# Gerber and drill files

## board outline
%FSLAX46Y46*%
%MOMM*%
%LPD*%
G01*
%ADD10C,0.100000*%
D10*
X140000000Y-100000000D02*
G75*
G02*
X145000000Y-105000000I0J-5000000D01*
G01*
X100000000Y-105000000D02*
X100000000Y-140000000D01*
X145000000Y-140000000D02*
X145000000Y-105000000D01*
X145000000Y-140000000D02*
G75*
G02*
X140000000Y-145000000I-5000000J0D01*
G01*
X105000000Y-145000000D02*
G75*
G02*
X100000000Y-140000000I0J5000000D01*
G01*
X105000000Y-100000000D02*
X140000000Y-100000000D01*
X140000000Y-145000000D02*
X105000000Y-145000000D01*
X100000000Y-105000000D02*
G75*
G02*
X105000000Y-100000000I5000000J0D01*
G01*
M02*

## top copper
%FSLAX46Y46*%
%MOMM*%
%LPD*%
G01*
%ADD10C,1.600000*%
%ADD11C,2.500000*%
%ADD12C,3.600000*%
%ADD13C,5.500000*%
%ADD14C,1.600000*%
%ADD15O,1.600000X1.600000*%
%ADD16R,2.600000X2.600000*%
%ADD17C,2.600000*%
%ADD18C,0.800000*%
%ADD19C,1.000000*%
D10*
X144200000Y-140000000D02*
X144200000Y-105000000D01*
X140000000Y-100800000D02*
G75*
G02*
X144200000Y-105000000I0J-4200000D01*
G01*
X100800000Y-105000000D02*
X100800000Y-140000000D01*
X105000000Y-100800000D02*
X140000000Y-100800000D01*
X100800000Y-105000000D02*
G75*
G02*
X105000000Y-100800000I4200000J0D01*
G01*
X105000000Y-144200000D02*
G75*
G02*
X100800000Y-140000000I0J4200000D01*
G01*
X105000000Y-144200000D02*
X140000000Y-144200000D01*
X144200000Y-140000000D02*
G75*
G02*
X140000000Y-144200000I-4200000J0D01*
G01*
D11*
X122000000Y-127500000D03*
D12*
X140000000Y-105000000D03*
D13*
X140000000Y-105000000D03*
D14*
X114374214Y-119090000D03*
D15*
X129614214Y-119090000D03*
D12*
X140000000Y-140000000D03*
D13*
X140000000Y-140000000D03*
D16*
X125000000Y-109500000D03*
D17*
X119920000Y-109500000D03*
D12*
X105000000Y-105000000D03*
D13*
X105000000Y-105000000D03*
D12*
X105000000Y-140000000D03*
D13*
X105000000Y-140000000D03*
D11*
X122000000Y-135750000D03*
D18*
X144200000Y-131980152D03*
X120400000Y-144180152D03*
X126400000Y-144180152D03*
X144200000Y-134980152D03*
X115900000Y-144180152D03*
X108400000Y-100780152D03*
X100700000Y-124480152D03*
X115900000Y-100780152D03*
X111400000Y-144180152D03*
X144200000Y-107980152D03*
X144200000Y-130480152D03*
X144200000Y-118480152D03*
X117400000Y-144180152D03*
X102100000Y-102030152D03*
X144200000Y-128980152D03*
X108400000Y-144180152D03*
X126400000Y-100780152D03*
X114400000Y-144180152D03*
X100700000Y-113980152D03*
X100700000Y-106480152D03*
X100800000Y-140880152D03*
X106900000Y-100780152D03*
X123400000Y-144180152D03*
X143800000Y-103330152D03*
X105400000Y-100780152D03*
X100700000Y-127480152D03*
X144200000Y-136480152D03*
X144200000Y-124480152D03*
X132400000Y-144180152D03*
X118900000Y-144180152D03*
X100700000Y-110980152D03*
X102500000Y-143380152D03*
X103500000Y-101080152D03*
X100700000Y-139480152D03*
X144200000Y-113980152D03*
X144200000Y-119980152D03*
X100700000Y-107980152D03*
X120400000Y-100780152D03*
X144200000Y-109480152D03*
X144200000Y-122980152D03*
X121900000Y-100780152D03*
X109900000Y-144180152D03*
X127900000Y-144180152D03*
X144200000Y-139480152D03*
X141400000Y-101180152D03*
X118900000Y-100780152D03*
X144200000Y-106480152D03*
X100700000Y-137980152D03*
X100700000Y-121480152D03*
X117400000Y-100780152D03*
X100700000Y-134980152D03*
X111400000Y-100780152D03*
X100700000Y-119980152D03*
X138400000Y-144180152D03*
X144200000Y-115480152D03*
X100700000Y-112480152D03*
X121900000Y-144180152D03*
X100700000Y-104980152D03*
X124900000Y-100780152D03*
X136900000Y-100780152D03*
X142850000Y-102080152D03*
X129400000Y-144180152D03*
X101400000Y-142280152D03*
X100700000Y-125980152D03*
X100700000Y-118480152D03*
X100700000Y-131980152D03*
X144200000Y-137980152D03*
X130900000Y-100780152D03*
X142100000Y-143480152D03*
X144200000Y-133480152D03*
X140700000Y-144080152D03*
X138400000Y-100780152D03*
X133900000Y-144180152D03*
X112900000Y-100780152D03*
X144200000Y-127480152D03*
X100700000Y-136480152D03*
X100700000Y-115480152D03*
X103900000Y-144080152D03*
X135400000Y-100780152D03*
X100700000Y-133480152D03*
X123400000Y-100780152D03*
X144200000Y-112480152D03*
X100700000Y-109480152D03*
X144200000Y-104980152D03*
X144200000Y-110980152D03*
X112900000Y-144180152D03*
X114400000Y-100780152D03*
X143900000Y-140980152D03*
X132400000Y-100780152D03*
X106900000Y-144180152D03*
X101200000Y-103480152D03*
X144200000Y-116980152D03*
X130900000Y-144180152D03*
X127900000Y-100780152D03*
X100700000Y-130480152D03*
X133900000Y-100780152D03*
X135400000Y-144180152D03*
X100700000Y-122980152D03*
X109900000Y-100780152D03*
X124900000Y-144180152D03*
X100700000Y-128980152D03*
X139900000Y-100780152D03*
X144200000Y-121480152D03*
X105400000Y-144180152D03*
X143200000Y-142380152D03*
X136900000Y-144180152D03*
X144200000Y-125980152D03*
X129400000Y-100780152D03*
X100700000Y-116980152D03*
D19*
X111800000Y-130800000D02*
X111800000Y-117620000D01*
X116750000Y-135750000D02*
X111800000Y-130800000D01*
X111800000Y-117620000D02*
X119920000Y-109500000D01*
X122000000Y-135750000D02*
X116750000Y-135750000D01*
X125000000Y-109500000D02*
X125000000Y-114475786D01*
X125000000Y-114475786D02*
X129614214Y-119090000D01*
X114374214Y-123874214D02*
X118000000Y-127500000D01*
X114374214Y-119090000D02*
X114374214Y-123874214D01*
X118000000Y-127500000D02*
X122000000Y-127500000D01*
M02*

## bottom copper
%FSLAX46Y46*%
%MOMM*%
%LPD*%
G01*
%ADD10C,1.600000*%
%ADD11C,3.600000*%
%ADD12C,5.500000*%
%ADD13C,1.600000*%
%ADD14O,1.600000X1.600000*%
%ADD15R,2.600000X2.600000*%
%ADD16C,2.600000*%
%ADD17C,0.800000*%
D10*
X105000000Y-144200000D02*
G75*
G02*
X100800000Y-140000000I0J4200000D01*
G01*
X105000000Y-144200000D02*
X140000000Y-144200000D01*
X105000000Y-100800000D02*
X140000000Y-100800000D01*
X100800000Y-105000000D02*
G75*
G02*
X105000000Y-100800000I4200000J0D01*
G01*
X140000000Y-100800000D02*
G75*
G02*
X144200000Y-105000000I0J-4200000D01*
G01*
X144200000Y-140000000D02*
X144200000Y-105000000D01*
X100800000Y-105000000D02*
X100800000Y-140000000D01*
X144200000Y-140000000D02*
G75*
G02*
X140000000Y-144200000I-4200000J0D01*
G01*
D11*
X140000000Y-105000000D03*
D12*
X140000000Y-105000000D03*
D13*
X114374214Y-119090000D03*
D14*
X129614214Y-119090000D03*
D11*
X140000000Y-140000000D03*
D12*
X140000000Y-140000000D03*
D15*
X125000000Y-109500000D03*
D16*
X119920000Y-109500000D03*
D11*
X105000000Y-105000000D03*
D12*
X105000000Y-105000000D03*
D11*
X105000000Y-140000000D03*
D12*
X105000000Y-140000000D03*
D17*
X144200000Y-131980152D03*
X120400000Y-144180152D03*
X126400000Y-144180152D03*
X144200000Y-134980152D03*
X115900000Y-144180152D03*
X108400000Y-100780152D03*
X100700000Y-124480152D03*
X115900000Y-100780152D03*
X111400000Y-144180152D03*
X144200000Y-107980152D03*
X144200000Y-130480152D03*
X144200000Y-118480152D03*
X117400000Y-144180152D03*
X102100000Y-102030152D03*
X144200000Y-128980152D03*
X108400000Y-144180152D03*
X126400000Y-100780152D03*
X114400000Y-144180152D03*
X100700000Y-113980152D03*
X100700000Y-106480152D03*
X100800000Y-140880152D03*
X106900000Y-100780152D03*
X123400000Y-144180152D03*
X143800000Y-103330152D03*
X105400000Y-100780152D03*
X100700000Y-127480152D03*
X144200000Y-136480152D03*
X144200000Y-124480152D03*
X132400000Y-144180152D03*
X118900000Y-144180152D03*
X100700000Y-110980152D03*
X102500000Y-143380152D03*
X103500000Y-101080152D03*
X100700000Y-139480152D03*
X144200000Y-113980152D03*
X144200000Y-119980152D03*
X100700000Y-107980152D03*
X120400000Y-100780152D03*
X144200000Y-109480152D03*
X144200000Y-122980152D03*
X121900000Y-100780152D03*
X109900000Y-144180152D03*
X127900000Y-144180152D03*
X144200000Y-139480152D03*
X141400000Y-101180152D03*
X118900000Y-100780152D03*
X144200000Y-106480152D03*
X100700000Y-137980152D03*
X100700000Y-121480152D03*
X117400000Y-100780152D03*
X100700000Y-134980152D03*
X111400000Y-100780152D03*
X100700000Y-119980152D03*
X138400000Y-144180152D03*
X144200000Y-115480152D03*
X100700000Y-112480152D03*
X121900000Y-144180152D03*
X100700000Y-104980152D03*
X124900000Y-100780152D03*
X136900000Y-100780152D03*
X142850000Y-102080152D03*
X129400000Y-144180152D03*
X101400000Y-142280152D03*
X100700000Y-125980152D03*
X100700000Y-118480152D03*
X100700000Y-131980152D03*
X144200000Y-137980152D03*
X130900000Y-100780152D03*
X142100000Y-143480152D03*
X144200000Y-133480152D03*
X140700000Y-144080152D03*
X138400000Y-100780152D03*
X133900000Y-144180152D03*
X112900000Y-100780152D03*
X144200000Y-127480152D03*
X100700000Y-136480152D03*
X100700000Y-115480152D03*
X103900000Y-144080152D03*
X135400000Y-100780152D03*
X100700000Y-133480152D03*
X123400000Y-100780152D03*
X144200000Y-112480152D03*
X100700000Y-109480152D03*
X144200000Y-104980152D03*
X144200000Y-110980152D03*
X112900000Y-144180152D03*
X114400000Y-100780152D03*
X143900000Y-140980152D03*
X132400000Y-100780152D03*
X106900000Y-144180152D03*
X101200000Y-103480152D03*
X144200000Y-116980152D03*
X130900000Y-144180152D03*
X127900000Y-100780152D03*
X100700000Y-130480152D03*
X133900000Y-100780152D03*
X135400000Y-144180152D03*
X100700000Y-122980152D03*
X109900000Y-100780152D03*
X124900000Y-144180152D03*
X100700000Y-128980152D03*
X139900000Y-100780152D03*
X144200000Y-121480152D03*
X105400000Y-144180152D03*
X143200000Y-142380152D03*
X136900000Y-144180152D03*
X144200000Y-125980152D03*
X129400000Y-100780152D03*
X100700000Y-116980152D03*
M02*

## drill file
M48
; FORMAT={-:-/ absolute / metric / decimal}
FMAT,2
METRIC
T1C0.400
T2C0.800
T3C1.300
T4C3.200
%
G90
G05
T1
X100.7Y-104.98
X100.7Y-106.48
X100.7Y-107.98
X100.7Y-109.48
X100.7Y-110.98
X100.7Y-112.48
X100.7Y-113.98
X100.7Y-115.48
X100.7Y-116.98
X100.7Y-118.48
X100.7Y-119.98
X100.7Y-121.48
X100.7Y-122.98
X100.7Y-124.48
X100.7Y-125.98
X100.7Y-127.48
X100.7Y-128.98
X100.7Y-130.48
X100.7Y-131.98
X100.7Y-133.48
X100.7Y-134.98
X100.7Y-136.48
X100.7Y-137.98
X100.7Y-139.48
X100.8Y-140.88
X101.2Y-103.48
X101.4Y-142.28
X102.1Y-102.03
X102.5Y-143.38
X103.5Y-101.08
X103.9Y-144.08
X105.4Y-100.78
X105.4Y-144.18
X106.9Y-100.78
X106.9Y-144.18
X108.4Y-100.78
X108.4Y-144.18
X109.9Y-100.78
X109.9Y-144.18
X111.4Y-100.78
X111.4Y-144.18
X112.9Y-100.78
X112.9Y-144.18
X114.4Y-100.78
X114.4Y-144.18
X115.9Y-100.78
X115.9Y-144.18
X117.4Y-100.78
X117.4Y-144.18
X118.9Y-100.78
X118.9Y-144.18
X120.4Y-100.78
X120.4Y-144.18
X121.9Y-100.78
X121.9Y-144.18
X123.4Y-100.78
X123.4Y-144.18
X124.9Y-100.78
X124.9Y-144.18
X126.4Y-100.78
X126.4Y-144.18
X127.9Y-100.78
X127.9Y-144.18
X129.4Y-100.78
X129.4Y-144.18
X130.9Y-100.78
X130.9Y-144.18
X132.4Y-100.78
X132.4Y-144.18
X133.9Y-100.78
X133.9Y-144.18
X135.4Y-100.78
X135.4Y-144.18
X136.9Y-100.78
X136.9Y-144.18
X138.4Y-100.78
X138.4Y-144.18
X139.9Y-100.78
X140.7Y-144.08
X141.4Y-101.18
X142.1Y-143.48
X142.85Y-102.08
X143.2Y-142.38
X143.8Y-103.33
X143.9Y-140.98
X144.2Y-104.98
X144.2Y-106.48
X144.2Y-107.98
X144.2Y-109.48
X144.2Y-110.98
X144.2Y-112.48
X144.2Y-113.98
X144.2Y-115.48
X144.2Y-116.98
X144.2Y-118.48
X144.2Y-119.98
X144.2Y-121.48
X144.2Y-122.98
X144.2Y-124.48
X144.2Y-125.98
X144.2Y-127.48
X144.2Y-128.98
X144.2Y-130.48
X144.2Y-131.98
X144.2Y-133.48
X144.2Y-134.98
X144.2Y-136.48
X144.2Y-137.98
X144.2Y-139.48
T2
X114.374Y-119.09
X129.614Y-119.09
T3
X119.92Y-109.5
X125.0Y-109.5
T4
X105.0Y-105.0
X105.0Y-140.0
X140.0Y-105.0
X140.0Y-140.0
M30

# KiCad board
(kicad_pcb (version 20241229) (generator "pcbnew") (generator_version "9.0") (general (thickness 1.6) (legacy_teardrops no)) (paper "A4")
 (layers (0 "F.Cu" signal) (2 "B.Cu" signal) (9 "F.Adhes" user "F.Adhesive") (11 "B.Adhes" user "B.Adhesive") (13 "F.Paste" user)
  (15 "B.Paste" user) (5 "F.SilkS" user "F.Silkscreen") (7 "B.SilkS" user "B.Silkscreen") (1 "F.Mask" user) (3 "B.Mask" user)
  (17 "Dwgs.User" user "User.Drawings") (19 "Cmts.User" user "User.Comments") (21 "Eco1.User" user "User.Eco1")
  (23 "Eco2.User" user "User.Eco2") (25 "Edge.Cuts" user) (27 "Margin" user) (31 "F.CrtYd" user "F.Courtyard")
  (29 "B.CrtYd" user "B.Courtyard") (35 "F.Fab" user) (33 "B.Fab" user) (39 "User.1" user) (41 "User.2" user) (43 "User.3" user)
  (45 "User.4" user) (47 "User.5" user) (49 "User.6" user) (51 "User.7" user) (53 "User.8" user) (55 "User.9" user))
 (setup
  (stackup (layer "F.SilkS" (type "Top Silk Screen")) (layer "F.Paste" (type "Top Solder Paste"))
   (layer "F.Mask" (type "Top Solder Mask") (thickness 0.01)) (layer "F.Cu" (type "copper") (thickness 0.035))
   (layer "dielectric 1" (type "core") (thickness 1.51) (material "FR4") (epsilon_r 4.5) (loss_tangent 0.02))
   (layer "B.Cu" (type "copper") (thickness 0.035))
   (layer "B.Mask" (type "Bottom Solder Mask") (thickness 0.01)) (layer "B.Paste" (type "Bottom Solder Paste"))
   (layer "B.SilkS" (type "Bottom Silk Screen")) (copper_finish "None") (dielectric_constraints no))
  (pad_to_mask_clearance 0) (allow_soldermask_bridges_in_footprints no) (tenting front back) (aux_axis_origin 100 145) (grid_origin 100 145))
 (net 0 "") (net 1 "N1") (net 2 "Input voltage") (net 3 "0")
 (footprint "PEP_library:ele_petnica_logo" (layer "F.Cu") (at 136 126.6)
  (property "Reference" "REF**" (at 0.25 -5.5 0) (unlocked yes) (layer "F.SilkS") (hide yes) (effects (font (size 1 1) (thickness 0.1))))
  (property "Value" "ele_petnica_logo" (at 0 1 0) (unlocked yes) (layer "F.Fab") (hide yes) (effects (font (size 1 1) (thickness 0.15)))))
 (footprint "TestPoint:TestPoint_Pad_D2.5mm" (layer "F.Cu") (at 122 127.5)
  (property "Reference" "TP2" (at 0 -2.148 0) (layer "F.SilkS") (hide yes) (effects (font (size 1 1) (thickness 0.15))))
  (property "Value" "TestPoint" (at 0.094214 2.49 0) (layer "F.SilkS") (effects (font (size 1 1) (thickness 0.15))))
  (pad "1" smd circle (at 0 0) (size 2.5 2.5) (layers "F.Cu" "F.Mask") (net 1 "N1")))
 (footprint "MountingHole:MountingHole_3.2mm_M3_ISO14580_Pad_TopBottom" (layer "F.Cu") (at 140 105)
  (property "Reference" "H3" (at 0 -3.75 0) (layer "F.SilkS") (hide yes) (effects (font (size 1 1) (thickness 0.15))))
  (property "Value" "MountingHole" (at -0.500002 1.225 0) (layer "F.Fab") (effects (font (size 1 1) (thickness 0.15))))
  (pad "1" thru_hole circle (at 0 0) (size 3.6 3.6) (drill 3.2) (layers "*.Cu" "*.Mask") (remove_unused_layers no))
  (pad "1" connect circle (at 0 0) (size 5.5 5.5) (layers "F.Cu" "F.Mask"))
  (pad "1" connect circle (at 0 0) (size 5.5 5.5) (layers "B.Cu" "B.Mask")))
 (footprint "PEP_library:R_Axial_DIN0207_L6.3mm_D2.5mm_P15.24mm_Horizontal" (layer "F.Cu") (at 114.374214 119.09)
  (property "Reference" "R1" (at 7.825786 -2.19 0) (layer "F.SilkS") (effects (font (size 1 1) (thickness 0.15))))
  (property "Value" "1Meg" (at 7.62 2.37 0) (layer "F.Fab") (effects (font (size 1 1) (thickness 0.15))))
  (pad "1" thru_hole circle (at 0 0) (size 1.6 1.6) (drill 0.8) (layers "*.Cu" "*.Mask") (remove_unused_layers no) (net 1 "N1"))
  (pad "2" thru_hole oval (at 15.24 0) (size 1.6 1.6) (drill 0.8) (layers "*.Cu" "*.Mask") (remove_unused_layers no) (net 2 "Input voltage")))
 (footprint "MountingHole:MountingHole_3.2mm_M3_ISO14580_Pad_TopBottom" (layer "F.Cu") (at 140 140)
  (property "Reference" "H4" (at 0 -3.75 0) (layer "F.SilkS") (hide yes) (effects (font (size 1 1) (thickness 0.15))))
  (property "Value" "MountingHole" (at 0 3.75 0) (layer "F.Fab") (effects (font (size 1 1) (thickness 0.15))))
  (pad "1" thru_hole circle (at 0 0) (size 3.6 3.6) (drill 3.2) (layers "*.Cu" "*.Mask") (remove_unused_layers no))
  (pad "1" connect circle (at 0 0) (size 5.5 5.5) (layers "F.Cu" "F.Mask"))
  (pad "1" connect circle (at 0 0) (size 5.5 5.5) (layers "B.Cu" "B.Mask")))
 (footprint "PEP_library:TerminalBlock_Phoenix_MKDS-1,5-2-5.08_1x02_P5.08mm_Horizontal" (layer "F.Cu") (at 125 109.5 180)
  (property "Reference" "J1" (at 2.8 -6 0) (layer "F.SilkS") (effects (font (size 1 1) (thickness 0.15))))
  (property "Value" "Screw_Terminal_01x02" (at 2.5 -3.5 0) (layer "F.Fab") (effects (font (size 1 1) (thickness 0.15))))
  (pad "1" thru_hole rect (at 0 0 180) (size 2.6 2.6) (drill 1.3) (layers "*.Cu" "*.Mask") (remove_unused_layers no) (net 2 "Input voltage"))
  (pad "2" thru_hole circle (at 5.08 0 180) (size 2.6 2.6) (drill 1.3) (layers "*.Cu" "*.Mask") (remove_unused_layers no) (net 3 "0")))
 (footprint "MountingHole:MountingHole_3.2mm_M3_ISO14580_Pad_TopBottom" (layer "F.Cu") (at 105 105)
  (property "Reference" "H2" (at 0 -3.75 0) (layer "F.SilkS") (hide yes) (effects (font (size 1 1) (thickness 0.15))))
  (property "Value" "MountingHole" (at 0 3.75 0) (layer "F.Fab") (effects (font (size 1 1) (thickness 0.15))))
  (pad "1" thru_hole circle (at 0 0) (size 3.6 3.6) (drill 3.2) (layers "*.Cu" "*.Mask") (remove_unused_layers no))
  (pad "1" connect circle (at 0 0) (size 5.5 5.5) (layers "F.Cu" "F.Mask"))
  (pad "1" connect circle (at 0 0) (size 5.5 5.5) (layers "B.Cu" "B.Mask")))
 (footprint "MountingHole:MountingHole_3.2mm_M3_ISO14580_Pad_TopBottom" (layer "F.Cu") (at 105 140 -90)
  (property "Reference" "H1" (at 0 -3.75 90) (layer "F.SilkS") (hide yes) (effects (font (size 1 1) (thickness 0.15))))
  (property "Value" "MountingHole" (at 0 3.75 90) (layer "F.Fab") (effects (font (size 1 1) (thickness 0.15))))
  (pad "1" thru_hole circle (at 0 0 270) (size 3.6 3.6) (drill 3.2) (layers "*.Cu" "*.Mask") (remove_unused_layers no))
  (pad "1" connect circle (at 0 0 270) (size 5.5 5.5) (layers "F.Cu" "F.Mask"))
  (pad "1" connect circle (at 0 0 270) (size 5.5 5.5) (layers "B.Cu" "B.Mask")))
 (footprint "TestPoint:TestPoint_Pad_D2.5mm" (layer "F.Cu") (at 122 135.75)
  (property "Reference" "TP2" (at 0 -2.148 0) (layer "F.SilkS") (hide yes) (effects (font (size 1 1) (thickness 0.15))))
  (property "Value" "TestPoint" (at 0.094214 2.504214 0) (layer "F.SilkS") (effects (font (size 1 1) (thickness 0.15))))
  (pad "2" smd circle (at 0 0) (size 2.5 2.5) (layers "F.Cu" "F.Mask") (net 3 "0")))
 (gr_line (start 144.2 140) (end 144.2 105) (stroke (width 1.6) (type default)) (locked yes) (layer "F.Cu"))
 (gr_arc (start 140 100.8) (mid 142.969848 102.030152) (end 144.2 105) (stroke (width 1.6) (type default)) (locked yes) (layer "F.Cu"))
 (gr_line (start 100.8 105) (end 100.8 140) (stroke (width 1.6) (type default)) (locked yes) (layer "F.Cu"))
 (gr_line (start 105 100.8) (end 140 100.8) (stroke (width 1.6) (type default)) (locked yes) (layer "F.Cu"))
 (gr_arc (start 100.8 105) (mid 102.030152 102.030152) (end 105 100.8) (stroke (width 1.6) (type default)) (locked yes) (layer "F.Cu"))
 (gr_arc (start 105 144.2) (mid 102.030152 142.969848) (end 100.8 140) (stroke (width 1.6) (type default)) (locked yes) (layer "F.Cu"))
 (gr_line (start 105 144.2) (end 140 144.2) (stroke (width 1.6) (type default)) (locked yes) (layer "F.Cu"))
 (gr_arc (start 144.2 140) (mid 142.969848 142.969848) (end 140 144.2) (stroke (width 1.6) (type default)) (locked yes) (layer "F.Cu"))
 (gr_arc (start 105 144.2) (mid 102.030154 142.969848) (end 100.8 140) (stroke (width 1.6) (type default)) (locked yes) (layer "B.Cu"))
 (gr_line (start 105 144.2) (end 140 144.2) (stroke (width 1.6) (type default)) (locked yes) (layer "B.Cu"))
 (gr_line (start 105 100.8) (end 140 100.8) (stroke (width 1.6) (type default)) (locked yes) (layer "B.Cu"))
 (gr_arc (start 100.8 105) (mid 102.030152 102.030152) (end 105 100.8) (stroke (width 1.6) (type default)) (locked yes) (layer "B.Cu"))
 (gr_arc (start 140 100.8) (mid 142.96985 102.030151) (end 144.2 105) (stroke (width 1.6) (type default)) (locked yes) (layer "B.Cu"))
 (gr_line (start 144.2 140) (end 144.2 105) (stroke (width 1.6) (type default)) (locked yes) (layer "B.Cu"))
 (gr_line (start 100.8 105) (end 100.8 140) (stroke (width 1.6) (type default)) (locked yes) (layer "B.Cu"))
 (gr_arc (start 144.2 140) (mid 142.969849 142.969849) (end 140 144.2) (stroke (width 1.6) (type default)) (locked yes) (layer "B.Cu"))
 (gr_arc (start 140 100) (mid 143.535534 101.464466) (end 145 105) (stroke (width 0.1) (type default)) (locked yes) (layer "Edge.Cuts"))
 (gr_line (start 100 105) (end 100 140) (stroke (width 0.1) (type default)) (locked yes) (layer "Edge.Cuts"))
 (gr_line (start 145 140) (end 145 105) (stroke (width 0.1) (type default)) (locked yes) (layer "Edge.Cuts"))
 (gr_arc (start 145 140) (mid 143.535534 143.535534) (end 140 145) (stroke (width 0.1) (type default)) (locked yes) (layer "Edge.Cuts"))
 (gr_arc (start 105 145) (mid 101.464466 143.535534) (end 100 140) (stroke (width 0.1) (type default)) (locked yes) (layer "Edge.Cuts"))
 (gr_line (start 105 100) (end 140 100) (stroke (width 0.1) (type default)) (locked yes) (layer "Edge.Cuts"))
 (gr_line (start 140 145) (end 105 145) (stroke (width 0.1) (type default)) (locked yes) (layer "Edge.Cuts"))
 (gr_arc (start 100 105) (mid 101.464466 101.464466) (end 105 100) (stroke (width 0.1) (type default)) (locked yes) (layer "Edge.Cuts"))
 (via (at 144.2 131.980152) (size 0.8) (drill 0.4) (layers "F.Cu" "B.Cu") (locked yes) (free yes) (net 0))
 (via (at 120.4 144.180152) (size 0.8) (drill 0.4) (layers "F.Cu" "B.Cu") (locked yes) (free yes) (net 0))
 (via (at 126.4 144.180152) (size 0.8) (drill 0.4) (layers "F.Cu" "B.Cu") (locked yes) (free yes) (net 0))
 (via (at 144.2 134.980152) (size 0.8) (drill 0.4) (layers "F.Cu" "B.Cu") (locked yes) (free yes) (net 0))
 (via (at 115.9 144.180152) (size 0.8) (drill 0.4) (layers "F.Cu" "B.Cu") (locked yes) (free yes) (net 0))
 (via (at 108.4 100.780152) (size 0.8) (drill 0.4) (layers "F.Cu" "B.Cu") (locked yes) (free yes) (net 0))
 (via (at 100.7 124.480152) (size 0.8) (drill 0.4) (layers "F.Cu" "B.Cu") (locked yes) (free yes) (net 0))
 (via (at 115.9 100.780152) (size 0.8) (drill 0.4) (layers "F.Cu" "B.Cu") (locked yes) (free yes) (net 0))
 (via (at 111.4 144.180152) (size 0.8) (drill 0.4) (layers "F.Cu" "B.Cu") (locked yes) (free yes) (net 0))
 (via (at 144.2 107.980152) (size 0.8) (drill 0.4) (layers "F.Cu" "B.Cu") (locked yes) (free yes) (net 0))
 (via (at 144.2 130.480152) (size 0.8) (drill 0.4) (layers "F.Cu" "B.Cu") (locked yes) (free yes) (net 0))
 (via (at 144.2 118.480152) (size 0.8) (drill 0.4) (layers "F.Cu" "B.Cu") (locked yes) (free yes) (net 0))
 (via (at 117.4 144.180152) (size 0.8) (drill 0.4) (layers "F.Cu" "B.Cu") (locked yes) (free yes) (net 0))
 (via (at 102.1 102.030152) (size 0.8) (drill 0.4) (layers "F.Cu" "B.Cu") (locked yes) (free yes) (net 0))
 (via (at 144.2 128.980152) (size 0.8) (drill 0.4) (layers "F.Cu" "B.Cu") (locked yes) (free yes) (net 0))
 (via (at 108.4 144.180152) (size 0.8) (drill 0.4) (layers "F.Cu" "B.Cu") (locked yes) (free yes) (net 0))
 (via (at 126.4 100.780152) (size 0.8) (drill 0.4) (layers "F.Cu" "B.Cu") (locked yes) (free yes) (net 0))
 (via (at 114.4 144.180152) (size 0.8) (drill 0.4) (layers "F.Cu" "B.Cu") (locked yes) (free yes) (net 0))
 (via (at 100.7 113.980152) (size 0.8) (drill 0.4) (layers "F.Cu" "B.Cu") (locked yes) (free yes) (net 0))
 (via (at 100.7 106.480152) (size 0.8) (drill 0.4) (layers "F.Cu" "B.Cu") (locked yes) (free yes) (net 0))
 (via (at 100.8 140.880152) (size 0.8) (drill 0.4) (layers "F.Cu" "B.Cu") (locked yes) (free yes) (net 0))
 (via (at 106.9 100.780152) (size 0.8) (drill 0.4) (layers "F.Cu" "B.Cu") (locked yes) (free yes) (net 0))
 (via (at 123.4 144.180152) (size 0.8) (drill 0.4) (layers "F.Cu" "B.Cu") (locked yes) (free yes) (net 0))
 (via (at 143.8 103.330152) (size 0.8) (drill 0.4) (layers "F.Cu" "B.Cu") (locked yes) (free yes) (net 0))
 (via (at 105.4 100.780152) (size 0.8) (drill 0.4) (layers "F.Cu" "B.Cu") (locked yes) (free yes) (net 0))
 (via (at 100.7 127.480152) (size 0.8) (drill 0.4) (layers "F.Cu" "B.Cu") (locked yes) (free yes) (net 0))
 (via (at 144.2 136.480152) (size 0.8) (drill 0.4) (layers "F.Cu" "B.Cu") (locked yes) (free yes) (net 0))
 (via (at 144.2 124.480152) (size 0.8) (drill 0.4) (layers "F.Cu" "B.Cu") (locked yes) (free yes) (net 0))
 (via (at 132.4 144.180152) (size 0.8) (drill 0.4) (layers "F.Cu" "B.Cu") (locked yes) (free yes) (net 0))
 (via (at 118.9 144.180152) (size 0.8) (drill 0.4) (layers "F.Cu" "B.Cu") (locked yes) (free yes) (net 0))
 (via (at 100.7 110.980152) (size 0.8) (drill 0.4) (layers "F.Cu" "B.Cu") (locked yes) (free yes) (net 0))
 (via (at 102.5 143.380152) (size 0.8) (drill 0.4) (layers "F.Cu" "B.Cu") (locked yes) (free yes) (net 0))
 (via (at 103.5 101.080152) (size 0.8) (drill 0.4) (layers "F.Cu" "B.Cu") (locked yes) (free yes) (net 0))
 (via (at 100.7 139.480152) (size 0.8) (drill 0.4) (layers "F.Cu" "B.Cu") (locked yes) (free yes) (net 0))
 (via (at 144.2 113.980152) (size 0.8) (drill 0.4) (layers "F.Cu" "B.Cu") (locked yes) (free yes) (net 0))
 (via (at 144.2 119.980152) (size 0.8) (drill 0.4) (layers "F.Cu" "B.Cu") (locked yes) (free yes) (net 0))
 (via (at 100.7 107.980152) (size 0.8) (drill 0.4) (layers "F.Cu" "B.Cu") (locked yes) (free yes) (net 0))
 (via (at 120.4 100.780152) (size 0.8) (drill 0.4) (layers "F.Cu" "B.Cu") (locked yes) (free yes) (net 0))
 (via (at 144.2 109.480152) (size 0.8) (drill 0.4) (layers "F.Cu" "B.Cu") (locked yes) (free yes) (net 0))
 (via (at 144.2 122.980152) (size 0.8) (drill 0.4) (layers "F.Cu" "B.Cu") (locked yes) (free yes) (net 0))
 (via (at 121.9 100.780152) (size 0.8) (drill 0.4) (layers "F.Cu" "B.Cu") (locked yes) (free yes) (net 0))
 (via (at 109.9 144.180152) (size 0.8) (drill 0.4) (layers "F.Cu" "B.Cu") (locked yes) (free yes) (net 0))
 (via (at 127.9 144.180152) (size 0.8) (drill 0.4) (layers "F.Cu" "B.Cu") (locked yes) (free yes) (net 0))
 (via (at 144.2 139.480152) (size 0.8) (drill 0.4) (layers "F.Cu" "B.Cu") (locked yes) (free yes) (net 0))
 (via (at 141.4 101.180152) (size 0.8) (drill 0.4) (layers "F.Cu" "B.Cu") (locked yes) (free yes) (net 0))
 (via (at 118.9 100.780152) (size 0.8) (drill 0.4) (layers "F.Cu" "B.Cu") (locked yes) (free yes) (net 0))
 (via (at 144.2 106.480152) (size 0.8) (drill 0.4) (layers "F.Cu" "B.Cu") (locked yes) (free yes) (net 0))
 (via (at 100.7 137.980152) (size 0.8) (drill 0.4) (layers "F.Cu" "B.Cu") (locked yes) (free yes) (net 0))
 (via (at 100.7 121.480152) (size 0.8) (drill 0.4) (layers "F.Cu" "B.Cu") (locked yes) (free yes) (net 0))
 (via (at 117.4 100.780152) (size 0.8) (drill 0.4) (layers "F.Cu" "B.Cu") (locked yes) (free yes) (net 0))
 (via (at 100.7 134.980152) (size 0.8) (drill 0.4) (layers "F.Cu" "B.Cu") (locked yes) (free yes) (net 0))
 (via (at 111.4 100.780152) (size 0.8) (drill 0.4) (layers "F.Cu" "B.Cu") (locked yes) (free yes) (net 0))
 (via (at 100.7 119.980152) (size 0.8) (drill 0.4) (layers "F.Cu" "B.Cu") (locked yes) (free yes) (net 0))
 (via (at 138.4 144.180152) (size 0.8) (drill 0.4) (layers "F.Cu" "B.Cu") (locked yes) (free yes) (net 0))
 (via (at 144.2 115.480152) (size 0.8) (drill 0.4) (layers "F.Cu" "B.Cu") (locked yes) (free yes) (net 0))
 (via (at 100.7 112.480152) (size 0.8) (drill 0.4) (layers "F.Cu" "B.Cu") (locked yes) (free yes) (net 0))
 (via (at 121.9 144.180152) (size 0.8) (drill 0.4) (layers "F.Cu" "B.Cu") (locked yes) (free yes) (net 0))
 (via (at 100.7 104.980152) (size 0.8) (drill 0.4) (layers "F.Cu" "B.Cu") (locked yes) (free yes) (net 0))
 (via (at 124.9 100.780152) (size 0.8) (drill 0.4) (layers "F.Cu" "B.Cu") (locked yes) (free yes) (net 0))
 (via (at 136.9 100.780152) (size 0.8) (drill 0.4) (layers "F.Cu" "B.Cu") (locked yes) (free yes) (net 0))
 (via (at 142.85 102.080152) (size 0.8) (drill 0.4) (layers "F.Cu" "B.Cu") (locked yes) (free yes) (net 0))
 (via (at 129.4 144.180152) (size 0.8) (drill 0.4) (layers "F.Cu" "B.Cu") (locked yes) (free yes) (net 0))
 (via (at 101.4 142.280152) (size 0.8) (drill 0.4) (layers "F.Cu" "B.Cu") (locked yes) (free yes) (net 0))
 (via (at 100.7 125.980152) (size 0.8) (drill 0.4) (layers "F.Cu" "B.Cu") (locked yes) (free yes) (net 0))
 (via (at 100.7 118.480152) (size 0.8) (drill 0.4) (layers "F.Cu" "B.Cu") (locked yes) (free yes) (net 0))
 (via (at 100.7 131.980152) (size 0.8) (drill 0.4) (layers "F.Cu" "B.Cu") (locked yes) (free yes) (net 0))
 (via (at 144.2 137.980152) (size 0.8) (drill 0.4) (layers "F.Cu" "B.Cu") (locked yes) (free yes) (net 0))
 (via (at 130.9 100.780152) (size 0.8) (drill 0.4) (layers "F.Cu" "B.Cu") (locked yes) (free yes) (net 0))
 (via (at 142.1 143.480152) (size 0.8) (drill 0.4) (layers "F.Cu" "B.Cu") (locked yes) (free yes) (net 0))
 (via (at 144.2 133.480152) (size 0.8) (drill 0.4) (layers "F.Cu" "B.Cu") (locked yes) (free yes) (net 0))
 (via (at 140.7 144.080152) (size 0.8) (drill 0.4) (layers "F.Cu" "B.Cu") (locked yes) (free yes) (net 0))
 (via (at 138.4 100.780152) (size 0.8) (drill 0.4) (layers "F.Cu" "B.Cu") (locked yes) (free yes) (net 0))
 (via (at 133.9 144.180152) (size 0.8) (drill 0.4) (layers "F.Cu" "B.Cu") (locked yes) (free yes) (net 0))
 (via (at 112.9 100.780152) (size 0.8) (drill 0.4) (layers "F.Cu" "B.Cu") (locked yes) (free yes) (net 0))
 (via (at 144.2 127.480152) (size 0.8) (drill 0.4) (layers "F.Cu" "B.Cu") (locked yes) (free yes) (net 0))
 (via (at 100.7 136.480152) (size 0.8) (drill 0.4) (layers "F.Cu" "B.Cu") (locked yes) (free yes) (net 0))
 (via (at 100.7 115.480152) (size 0.8) (drill 0.4) (layers "F.Cu" "B.Cu") (locked yes) (free yes) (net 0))
 (via (at 103.9 144.080152) (size 0.8) (drill 0.4) (layers "F.Cu" "B.Cu") (locked yes) (free yes) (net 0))
 (via (at 135.4 100.780152) (size 0.8) (drill 0.4) (layers "F.Cu" "B.Cu") (locked yes) (free yes) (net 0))
 (via (at 100.7 133.480152) (size 0.8) (drill 0.4) (layers "F.Cu" "B.Cu") (locked yes) (free yes) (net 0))
 (via (at 123.4 100.780152) (size 0.8) (drill 0.4) (layers "F.Cu" "B.Cu") (locked yes) (free yes) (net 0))
 (via (at 144.2 112.480152) (size 0.8) (drill 0.4) (layers "F.Cu" "B.Cu") (locked yes) (free yes) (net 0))
 (via (at 100.7 109.480152) (size 0.8) (drill 0.4) (layers "F.Cu" "B.Cu") (locked yes) (free yes) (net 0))
 (via (at 144.2 104.980152) (size 0.8) (drill 0.4) (layers "F.Cu" "B.Cu") (locked yes) (free yes) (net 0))
 (via (at 144.2 110.980152) (size 0.8) (drill 0.4) (layers "F.Cu" "B.Cu") (locked yes) (free yes) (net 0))
 (via (at 112.9 144.180152) (size 0.8) (drill 0.4) (layers "F.Cu" "B.Cu") (locked yes) (free yes) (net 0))
 (via (at 114.4 100.780152) (size 0.8) (drill 0.4) (layers "F.Cu" "B.Cu") (locked yes) (free yes) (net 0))
 (via (at 143.9 140.980152) (size 0.8) (drill 0.4) (layers "F.Cu" "B.Cu") (locked yes) (free yes) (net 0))
 (via (at 132.4 100.780152) (size 0.8) (drill 0.4) (layers "F.Cu" "B.Cu") (locked yes) (free yes) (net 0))
 (via (at 106.9 144.180152) (size 0.8) (drill 0.4) (layers "F.Cu" "B.Cu") (locked yes) (free yes) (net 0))
 (via (at 101.2 103.480152) (size 0.8) (drill 0.4) (layers "F.Cu" "B.Cu") (locked yes) (free yes) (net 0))
 (via (at 144.2 116.980152) (size 0.8) (drill 0.4) (layers "F.Cu" "B.Cu") (locked yes) (free yes) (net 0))
 (via (at 130.9 144.180152) (size 0.8) (drill 0.4) (layers "F.Cu" "B.Cu") (locked yes) (free yes) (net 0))
 (via (at 127.9 100.780152) (size 0.8) (drill 0.4) (layers "F.Cu" "B.Cu") (locked yes) (free yes) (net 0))
 (via (at 100.7 130.480152) (size 0.8) (drill 0.4) (layers "F.Cu" "B.Cu") (locked yes) (free yes) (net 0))
 (via (at 133.9 100.780152) (size 0.8) (drill 0.4) (layers "F.Cu" "B.Cu") (locked yes) (free yes) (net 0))
 (via (at 135.4 144.180152) (size 0.8) (drill 0.4) (layers "F.Cu" "B.Cu") (locked yes) (free yes) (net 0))
 (via (at 100.7 122.980152) (size 0.8) (drill 0.4) (layers "F.Cu" "B.Cu") (locked yes) (free yes) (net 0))
 (via (at 109.9 100.780152) (size 0.8) (drill 0.4) (layers "F.Cu" "B.Cu") (locked yes) (free yes) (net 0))
 (via (at 124.9 144.180152) (size 0.8) (drill 0.4) (layers "F.Cu" "B.Cu") (locked yes) (free yes) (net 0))
 (via (at 100.7 128.980152) (size 0.8) (drill 0.4) (layers "F.Cu" "B.Cu") (locked yes) (free yes) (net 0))
 (via (at 139.9 100.780152) (size 0.8) (drill 0.4) (layers "F.Cu" "B.Cu") (locked yes) (free yes) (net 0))
 (via (at 144.2 121.480152) (size 0.8) (drill 0.4) (layers "F.Cu" "B.Cu") (locked yes) (free yes) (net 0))
 (via (at 105.4 144.180152) (size 0.8) (drill 0.4) (layers "F.Cu" "B.Cu") (locked yes) (free yes) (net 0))
 (via (at 143.2 142.380152) (size 0.8) (drill 0.4) (layers "F.Cu" "B.Cu") (locked yes) (free yes) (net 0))
 (via (at 136.9 144.180152) (size 0.8) (drill 0.4) (layers "F.Cu" "B.Cu") (locked yes) (free yes) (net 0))
 (via (at 144.2 125.980152) (size 0.8) (drill 0.4) (layers "F.Cu" "B.Cu") (locked yes) (free yes) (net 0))
 (via (at 129.4 100.780152) (size 0.8) (drill 0.4) (layers "F.Cu" "B.Cu") (locked yes) (free yes) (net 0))
 (via (at 100.7 116.980152) (size 0.8) (drill 0.4) (layers "F.Cu" "B.Cu") (locked yes) (free yes) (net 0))
 (segment (start 111.8 130.8) (end 111.8 117.62) (width 1) (layer "F.Cu") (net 3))
 (segment (start 116.75 135.75) (end 111.8 130.8) (width 1) (layer "F.Cu") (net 3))
 (segment (start 111.8 117.62) (end 119.92 109.5) (width 1) (layer "F.Cu") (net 3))
 (segment (start 122 135.75) (end 116.75 135.75) (width 1) (layer "F.Cu") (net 3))
 (segment (start 125 109.5) (end 125 114.475786) (width 1) (layer "F.Cu") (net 2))
 (segment (start 125 114.475786) (end 129.614214 119.09) (width 1) (layer "F.Cu") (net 2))
 (segment (start 114.374214 123.874214) (end 118 127.5) (width 1) (layer "F.Cu") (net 1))
 (segment (start 114.374214 119.09) (end 114.374214 123.874214) (width 1) (layer "F.Cu") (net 1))
 (segment (start 118 127.5) (end 122 127.5) (width 1) (layer "F.Cu") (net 1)))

